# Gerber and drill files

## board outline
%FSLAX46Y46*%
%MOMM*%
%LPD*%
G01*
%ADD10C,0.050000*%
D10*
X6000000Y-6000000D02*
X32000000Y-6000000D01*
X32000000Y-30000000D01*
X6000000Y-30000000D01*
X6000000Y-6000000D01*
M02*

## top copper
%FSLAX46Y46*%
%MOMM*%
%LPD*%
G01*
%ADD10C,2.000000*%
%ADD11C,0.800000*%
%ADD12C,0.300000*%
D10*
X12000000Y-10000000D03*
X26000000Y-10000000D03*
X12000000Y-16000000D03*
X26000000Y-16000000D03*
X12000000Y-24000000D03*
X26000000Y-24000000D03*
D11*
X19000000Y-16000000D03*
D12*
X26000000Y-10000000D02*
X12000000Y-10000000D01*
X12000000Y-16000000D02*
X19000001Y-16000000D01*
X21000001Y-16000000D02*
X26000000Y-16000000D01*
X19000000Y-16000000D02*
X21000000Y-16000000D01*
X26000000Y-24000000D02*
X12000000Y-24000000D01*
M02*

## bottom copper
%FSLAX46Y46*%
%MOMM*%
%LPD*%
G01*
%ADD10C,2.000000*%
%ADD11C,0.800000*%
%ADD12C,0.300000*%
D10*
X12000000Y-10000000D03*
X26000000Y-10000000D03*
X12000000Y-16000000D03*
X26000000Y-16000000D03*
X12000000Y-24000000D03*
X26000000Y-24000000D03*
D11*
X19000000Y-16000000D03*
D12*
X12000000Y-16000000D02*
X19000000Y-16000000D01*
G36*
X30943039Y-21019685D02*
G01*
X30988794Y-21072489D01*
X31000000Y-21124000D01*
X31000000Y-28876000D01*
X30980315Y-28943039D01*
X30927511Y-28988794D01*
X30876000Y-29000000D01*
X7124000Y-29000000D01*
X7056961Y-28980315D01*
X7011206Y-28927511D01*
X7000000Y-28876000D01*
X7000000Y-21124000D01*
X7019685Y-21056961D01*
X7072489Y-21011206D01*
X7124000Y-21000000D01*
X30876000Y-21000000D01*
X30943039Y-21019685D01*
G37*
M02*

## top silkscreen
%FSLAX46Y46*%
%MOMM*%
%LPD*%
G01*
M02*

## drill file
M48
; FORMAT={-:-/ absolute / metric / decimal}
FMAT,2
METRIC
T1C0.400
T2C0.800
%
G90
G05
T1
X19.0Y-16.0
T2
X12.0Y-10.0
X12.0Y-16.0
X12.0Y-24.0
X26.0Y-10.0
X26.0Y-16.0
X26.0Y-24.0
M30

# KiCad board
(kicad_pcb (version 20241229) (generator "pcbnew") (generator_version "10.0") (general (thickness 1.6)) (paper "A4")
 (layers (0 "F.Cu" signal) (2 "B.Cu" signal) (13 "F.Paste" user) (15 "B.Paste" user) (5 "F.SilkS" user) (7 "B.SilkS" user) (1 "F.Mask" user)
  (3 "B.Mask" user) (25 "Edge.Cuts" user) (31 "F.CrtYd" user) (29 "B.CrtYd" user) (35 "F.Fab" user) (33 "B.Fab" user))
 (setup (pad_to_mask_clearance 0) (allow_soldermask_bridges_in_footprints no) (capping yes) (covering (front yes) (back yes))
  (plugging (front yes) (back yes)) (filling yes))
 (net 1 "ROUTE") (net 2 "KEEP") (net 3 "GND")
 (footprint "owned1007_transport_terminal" (layer "F.Cu") (at 12 10)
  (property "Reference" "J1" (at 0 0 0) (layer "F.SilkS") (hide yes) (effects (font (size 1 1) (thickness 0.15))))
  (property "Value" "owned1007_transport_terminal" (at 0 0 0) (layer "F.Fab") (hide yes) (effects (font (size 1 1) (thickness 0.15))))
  (pad "1" thru_hole circle (at 0 0) (size 2 2) (drill 0.8) (layers "*.Cu" "*.Mask") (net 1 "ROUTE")))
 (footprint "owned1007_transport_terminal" (layer "F.Cu") (at 26 10)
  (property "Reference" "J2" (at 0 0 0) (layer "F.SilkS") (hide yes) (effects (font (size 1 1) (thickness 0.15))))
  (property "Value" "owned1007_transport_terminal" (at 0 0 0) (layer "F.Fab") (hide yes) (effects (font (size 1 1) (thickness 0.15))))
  (pad "1" thru_hole circle (at 0 0) (size 2 2) (drill 0.8) (layers "*.Cu" "*.Mask") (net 1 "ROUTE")))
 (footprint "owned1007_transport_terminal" (layer "F.Cu") (at 12 16)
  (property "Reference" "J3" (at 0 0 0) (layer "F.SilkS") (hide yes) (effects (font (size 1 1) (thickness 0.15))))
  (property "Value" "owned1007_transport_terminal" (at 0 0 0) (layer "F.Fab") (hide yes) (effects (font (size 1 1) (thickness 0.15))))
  (pad "1" thru_hole circle (at 0 0) (size 2 2) (drill 0.8) (layers "*.Cu" "*.Mask") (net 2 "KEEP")))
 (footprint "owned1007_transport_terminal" (layer "F.Cu") (at 26 16)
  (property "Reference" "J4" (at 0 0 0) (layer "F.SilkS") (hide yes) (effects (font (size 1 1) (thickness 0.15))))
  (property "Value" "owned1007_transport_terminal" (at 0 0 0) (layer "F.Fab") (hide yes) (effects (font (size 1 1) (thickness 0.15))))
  (pad "1" thru_hole circle (at 0 0) (size 2 2) (drill 0.8) (layers "*.Cu" "*.Mask") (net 2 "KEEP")))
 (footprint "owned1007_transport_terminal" (layer "F.Cu") (at 12 24)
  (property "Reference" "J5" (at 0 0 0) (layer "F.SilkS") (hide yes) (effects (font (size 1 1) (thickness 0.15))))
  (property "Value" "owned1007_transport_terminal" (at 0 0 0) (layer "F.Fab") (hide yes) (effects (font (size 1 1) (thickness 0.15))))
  (pad "1" thru_hole circle (at 0 0) (size 2 2) (drill 0.8) (layers "*.Cu" "*.Mask") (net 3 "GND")))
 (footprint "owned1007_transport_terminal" (layer "F.Cu") (at 26 24)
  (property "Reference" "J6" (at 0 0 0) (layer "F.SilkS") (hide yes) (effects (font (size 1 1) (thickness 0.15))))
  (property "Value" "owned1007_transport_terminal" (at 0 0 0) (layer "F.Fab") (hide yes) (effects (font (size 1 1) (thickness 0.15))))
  (pad "1" thru_hole circle (at 0 0) (size 2 2) (drill 0.8) (layers "*.Cu" "*.Mask") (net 3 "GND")))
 (gr_rect (start 6 6) (end 32 30) (stroke (width 0.05) (type default)) (fill none) (layer "Edge.Cuts"))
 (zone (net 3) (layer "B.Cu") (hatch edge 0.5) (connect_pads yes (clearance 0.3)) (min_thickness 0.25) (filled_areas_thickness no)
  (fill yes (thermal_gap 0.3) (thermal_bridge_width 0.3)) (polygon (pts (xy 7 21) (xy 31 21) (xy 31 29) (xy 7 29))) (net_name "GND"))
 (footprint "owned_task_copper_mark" (layer "F.Cu") (at 10 28)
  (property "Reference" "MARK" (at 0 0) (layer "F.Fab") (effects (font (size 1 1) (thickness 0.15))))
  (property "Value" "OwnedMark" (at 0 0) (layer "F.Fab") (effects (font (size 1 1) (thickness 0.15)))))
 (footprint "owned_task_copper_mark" (layer "F.Cu") (at 13 28)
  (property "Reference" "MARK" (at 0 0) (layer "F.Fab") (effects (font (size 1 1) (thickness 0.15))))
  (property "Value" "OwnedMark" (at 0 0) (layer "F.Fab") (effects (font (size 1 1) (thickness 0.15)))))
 (segment (start 26 10) (end 12 10) (width 0.3) (layer "F.Cu") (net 1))
 (segment (start 12 16) (end 19.000001 16) (width 0.3) (layer "F.Cu") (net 2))
 (segment (start 21.000001 16) (end 26 16) (width 0.3) (layer "F.Cu") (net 2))
 (segment (start 19 16) (end 21 16) (width 0.3) (layer "F.Cu") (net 2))
 (via (at 19 16) (size 0.8) (drill 0.4) (layers "F.Cu" "B.Cu") (free yes) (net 2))
 (segment (start 12 16) (end 19 16) (width 0.3) (layer "B.Cu") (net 2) (locked yes))
 (segment (start 26 24) (end 12 24) (width 0.3) (layer "F.Cu") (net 3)))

